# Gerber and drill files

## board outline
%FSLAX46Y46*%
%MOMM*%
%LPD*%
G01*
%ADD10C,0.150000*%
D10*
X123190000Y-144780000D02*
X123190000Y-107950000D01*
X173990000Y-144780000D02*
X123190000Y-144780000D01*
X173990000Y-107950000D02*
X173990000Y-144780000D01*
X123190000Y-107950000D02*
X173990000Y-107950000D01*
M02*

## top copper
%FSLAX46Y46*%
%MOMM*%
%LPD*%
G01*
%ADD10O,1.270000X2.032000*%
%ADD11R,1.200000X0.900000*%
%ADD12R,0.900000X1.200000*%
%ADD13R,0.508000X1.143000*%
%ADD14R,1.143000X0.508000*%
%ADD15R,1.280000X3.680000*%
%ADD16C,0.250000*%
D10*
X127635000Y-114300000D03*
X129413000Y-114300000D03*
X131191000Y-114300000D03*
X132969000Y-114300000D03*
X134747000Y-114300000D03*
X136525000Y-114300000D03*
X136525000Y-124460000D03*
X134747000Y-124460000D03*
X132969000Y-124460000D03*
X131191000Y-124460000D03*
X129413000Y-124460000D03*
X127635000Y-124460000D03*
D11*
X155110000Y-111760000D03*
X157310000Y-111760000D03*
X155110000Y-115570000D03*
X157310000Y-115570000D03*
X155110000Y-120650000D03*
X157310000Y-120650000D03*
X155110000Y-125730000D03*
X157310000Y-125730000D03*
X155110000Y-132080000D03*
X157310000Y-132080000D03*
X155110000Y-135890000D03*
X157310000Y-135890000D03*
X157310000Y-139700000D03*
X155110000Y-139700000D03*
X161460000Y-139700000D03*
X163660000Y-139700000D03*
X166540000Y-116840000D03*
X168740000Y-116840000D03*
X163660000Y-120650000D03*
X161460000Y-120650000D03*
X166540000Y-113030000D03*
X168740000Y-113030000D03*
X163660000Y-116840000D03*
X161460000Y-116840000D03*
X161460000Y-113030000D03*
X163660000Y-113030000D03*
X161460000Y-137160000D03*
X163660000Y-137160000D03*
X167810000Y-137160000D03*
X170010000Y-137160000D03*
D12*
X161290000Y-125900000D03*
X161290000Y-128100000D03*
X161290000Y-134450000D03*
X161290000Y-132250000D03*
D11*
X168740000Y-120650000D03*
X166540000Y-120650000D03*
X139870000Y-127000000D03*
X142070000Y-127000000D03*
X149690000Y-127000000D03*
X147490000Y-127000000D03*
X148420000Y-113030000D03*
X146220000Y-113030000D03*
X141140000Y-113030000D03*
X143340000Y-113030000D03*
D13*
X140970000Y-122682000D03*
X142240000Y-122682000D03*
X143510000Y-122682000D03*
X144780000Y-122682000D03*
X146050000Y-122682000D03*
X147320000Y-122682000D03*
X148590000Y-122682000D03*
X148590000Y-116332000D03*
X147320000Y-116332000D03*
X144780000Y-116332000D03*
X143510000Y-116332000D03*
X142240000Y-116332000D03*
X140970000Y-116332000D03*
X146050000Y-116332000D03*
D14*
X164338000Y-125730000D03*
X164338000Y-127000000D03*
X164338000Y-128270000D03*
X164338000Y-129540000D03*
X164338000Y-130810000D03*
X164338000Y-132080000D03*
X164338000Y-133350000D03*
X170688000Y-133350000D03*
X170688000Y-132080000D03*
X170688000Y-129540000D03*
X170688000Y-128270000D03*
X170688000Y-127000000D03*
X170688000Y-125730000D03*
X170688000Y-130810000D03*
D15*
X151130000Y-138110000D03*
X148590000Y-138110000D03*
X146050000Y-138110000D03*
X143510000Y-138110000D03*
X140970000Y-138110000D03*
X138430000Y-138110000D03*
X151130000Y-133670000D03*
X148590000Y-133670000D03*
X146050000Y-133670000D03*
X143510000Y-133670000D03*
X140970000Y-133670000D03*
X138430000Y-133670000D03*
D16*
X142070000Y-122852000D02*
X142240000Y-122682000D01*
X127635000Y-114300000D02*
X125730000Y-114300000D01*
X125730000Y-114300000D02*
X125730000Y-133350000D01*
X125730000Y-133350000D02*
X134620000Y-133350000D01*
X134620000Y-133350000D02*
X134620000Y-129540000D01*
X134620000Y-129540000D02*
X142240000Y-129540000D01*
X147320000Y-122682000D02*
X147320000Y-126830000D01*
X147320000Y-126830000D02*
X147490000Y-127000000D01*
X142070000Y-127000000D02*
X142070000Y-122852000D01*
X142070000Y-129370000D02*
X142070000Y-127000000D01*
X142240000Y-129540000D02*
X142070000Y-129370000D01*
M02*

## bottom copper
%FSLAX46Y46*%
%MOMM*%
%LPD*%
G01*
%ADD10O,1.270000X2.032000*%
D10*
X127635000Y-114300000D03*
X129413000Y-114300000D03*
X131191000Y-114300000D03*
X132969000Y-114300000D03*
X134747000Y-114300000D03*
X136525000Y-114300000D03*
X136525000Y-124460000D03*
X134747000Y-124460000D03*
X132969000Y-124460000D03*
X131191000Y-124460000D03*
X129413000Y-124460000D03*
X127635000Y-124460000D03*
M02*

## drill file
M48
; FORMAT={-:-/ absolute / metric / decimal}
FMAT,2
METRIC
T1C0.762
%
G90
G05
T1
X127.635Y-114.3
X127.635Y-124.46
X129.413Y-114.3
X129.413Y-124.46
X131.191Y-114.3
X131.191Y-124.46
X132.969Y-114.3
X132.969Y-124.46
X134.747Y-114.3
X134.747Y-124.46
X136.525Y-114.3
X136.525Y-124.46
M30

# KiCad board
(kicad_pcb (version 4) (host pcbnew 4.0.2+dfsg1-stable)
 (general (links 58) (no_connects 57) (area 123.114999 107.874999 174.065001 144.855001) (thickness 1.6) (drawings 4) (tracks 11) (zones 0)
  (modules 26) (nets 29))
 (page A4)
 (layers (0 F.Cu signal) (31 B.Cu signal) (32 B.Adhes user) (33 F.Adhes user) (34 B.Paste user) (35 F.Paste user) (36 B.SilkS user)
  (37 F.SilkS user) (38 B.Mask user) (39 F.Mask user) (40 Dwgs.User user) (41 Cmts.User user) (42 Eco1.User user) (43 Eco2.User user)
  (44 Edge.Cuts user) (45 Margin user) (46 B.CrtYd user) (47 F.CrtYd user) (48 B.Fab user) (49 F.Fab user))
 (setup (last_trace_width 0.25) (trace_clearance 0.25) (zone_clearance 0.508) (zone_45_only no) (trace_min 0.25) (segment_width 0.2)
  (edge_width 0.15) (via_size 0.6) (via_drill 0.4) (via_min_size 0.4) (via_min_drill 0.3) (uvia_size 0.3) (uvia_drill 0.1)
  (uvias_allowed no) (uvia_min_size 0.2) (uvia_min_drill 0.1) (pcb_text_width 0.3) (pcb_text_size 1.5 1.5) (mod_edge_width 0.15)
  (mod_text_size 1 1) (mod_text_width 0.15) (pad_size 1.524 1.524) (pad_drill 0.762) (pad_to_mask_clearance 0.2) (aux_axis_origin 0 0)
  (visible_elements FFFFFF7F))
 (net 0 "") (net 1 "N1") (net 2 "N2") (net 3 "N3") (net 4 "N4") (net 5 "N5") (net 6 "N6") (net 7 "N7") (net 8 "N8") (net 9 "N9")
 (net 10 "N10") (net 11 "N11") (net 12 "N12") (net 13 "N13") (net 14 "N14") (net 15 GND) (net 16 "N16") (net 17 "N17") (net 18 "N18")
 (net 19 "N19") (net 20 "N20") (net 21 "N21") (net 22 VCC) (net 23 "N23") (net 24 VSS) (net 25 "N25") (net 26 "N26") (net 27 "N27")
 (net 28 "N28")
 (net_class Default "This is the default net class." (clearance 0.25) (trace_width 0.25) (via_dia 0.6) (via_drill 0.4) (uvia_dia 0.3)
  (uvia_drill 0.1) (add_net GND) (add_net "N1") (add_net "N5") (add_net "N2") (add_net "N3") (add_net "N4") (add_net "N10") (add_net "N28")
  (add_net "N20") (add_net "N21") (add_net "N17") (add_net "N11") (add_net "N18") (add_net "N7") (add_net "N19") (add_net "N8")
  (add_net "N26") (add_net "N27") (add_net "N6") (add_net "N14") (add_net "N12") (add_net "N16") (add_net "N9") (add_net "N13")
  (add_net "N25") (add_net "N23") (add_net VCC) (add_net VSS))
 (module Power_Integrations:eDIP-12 (layer F.Cu) (at 132.08 119.38)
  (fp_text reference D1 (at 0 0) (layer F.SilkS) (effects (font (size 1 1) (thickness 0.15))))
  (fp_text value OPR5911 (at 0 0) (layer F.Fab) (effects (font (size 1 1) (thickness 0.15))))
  (pad 1 thru_hole oval (at -4.445 -5.08) (size 1.27 2.032) (drill 0.762) (layers *.Cu *.Mask F.SilkS) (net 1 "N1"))
  (pad 2 thru_hole oval (at -2.667 -5.08) (size 1.27 2.032) (drill 0.762) (layers *.Cu *.Mask F.SilkS) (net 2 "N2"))
  (pad 3 thru_hole oval (at -0.889 -5.08) (size 1.27 2.032) (drill 0.762) (layers *.Cu *.Mask F.SilkS))
  (pad 4 thru_hole oval (at 0.889 -5.08) (size 1.27 2.032) (drill 0.762) (layers *.Cu *.Mask F.SilkS))
  (pad 5 thru_hole oval (at 2.667 -5.08) (size 1.27 2.032) (drill 0.762) (layers *.Cu *.Mask F.SilkS))
  (pad 6 thru_hole oval (at 4.445 -5.08) (size 1.27 2.032) (drill 0.762) (layers *.Cu *.Mask F.SilkS) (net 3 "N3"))
  (pad 7 thru_hole oval (at 4.445 5.08) (size 1.27 2.032) (drill 0.762) (layers *.Cu *.Mask F.SilkS) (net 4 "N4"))
  (pad 8 thru_hole oval (at 2.667 5.08) (size 1.27 2.032) (drill 0.762) (layers *.Cu *.Mask F.SilkS))
  (pad 9 thru_hole oval (at 0.889 5.08) (size 1.27 2.032) (drill 0.762) (layers *.Cu *.Mask F.SilkS))
  (pad 10 thru_hole oval (at -0.889 5.08) (size 1.27 2.032) (drill 0.762) (layers *.Cu *.Mask F.SilkS))
  (pad 11 thru_hole oval (at -2.667 5.08) (size 1.27 2.032) (drill 0.762) (layers *.Cu *.Mask F.SilkS))
  (pad 12 thru_hole oval (at -4.445 5.08) (size 1.27 2.032) (drill 0.762) (layers *.Cu *.Mask F.SilkS) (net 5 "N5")))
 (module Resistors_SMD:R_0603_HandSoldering (layer F.Cu) (at 156.21 111.76)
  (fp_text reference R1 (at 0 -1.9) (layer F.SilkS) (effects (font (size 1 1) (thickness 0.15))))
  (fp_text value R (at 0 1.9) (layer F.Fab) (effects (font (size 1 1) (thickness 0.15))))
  (pad 1 smd rect (at -1.1 0) (size 1.2 0.9) (layers F.Cu F.Paste F.Mask) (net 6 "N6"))
  (pad 2 smd rect (at 1.1 0) (size 1.2 0.9) (layers F.Cu F.Paste F.Mask) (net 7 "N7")))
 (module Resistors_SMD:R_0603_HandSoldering (layer F.Cu) (at 156.21 115.57)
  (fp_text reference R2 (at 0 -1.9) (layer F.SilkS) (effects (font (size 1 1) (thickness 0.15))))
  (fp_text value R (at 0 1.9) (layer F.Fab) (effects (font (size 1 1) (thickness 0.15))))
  (pad 1 smd rect (at -1.1 0) (size 1.2 0.9) (layers F.Cu F.Paste F.Mask) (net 6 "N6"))
  (pad 2 smd rect (at 1.1 0) (size 1.2 0.9) (layers F.Cu F.Paste F.Mask) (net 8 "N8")))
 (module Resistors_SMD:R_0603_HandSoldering (layer F.Cu) (at 156.21 120.65)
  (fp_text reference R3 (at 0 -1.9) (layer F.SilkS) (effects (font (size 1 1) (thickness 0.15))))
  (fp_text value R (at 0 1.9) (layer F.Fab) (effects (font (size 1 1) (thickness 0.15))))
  (pad 1 smd rect (at -1.1 0) (size 1.2 0.9) (layers F.Cu F.Paste F.Mask) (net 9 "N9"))
  (pad 2 smd rect (at 1.1 0) (size 1.2 0.9) (layers F.Cu F.Paste F.Mask) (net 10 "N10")))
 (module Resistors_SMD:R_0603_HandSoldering (layer F.Cu) (at 156.21 125.73)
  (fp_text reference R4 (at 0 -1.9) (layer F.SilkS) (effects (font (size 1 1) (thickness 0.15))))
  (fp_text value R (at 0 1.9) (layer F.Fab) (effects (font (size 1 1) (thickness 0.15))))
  (pad 1 smd rect (at -1.1 0) (size 1.2 0.9) (layers F.Cu F.Paste F.Mask) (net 9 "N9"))
  (pad 2 smd rect (at 1.1 0) (size 1.2 0.9) (layers F.Cu F.Paste F.Mask) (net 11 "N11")))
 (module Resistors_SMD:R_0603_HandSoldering (layer F.Cu) (at 156.21 132.08)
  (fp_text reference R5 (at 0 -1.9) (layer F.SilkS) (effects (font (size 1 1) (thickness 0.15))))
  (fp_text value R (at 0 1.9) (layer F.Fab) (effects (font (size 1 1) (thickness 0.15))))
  (pad 1 smd rect (at -1.1 0) (size 1.2 0.9) (layers F.Cu F.Paste F.Mask) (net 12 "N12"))
  (pad 2 smd rect (at 1.1 0) (size 1.2 0.9) (layers F.Cu F.Paste F.Mask) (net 11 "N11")))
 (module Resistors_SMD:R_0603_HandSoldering (layer F.Cu) (at 156.21 135.89)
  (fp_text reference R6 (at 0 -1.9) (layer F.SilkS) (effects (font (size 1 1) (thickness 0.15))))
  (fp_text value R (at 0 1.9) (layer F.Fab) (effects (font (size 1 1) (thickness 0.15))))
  (pad 1 smd rect (at -1.1 0) (size 1.2 0.9) (layers F.Cu F.Paste F.Mask) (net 12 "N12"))
  (pad 2 smd rect (at 1.1 0) (size 1.2 0.9) (layers F.Cu F.Paste F.Mask) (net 7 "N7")))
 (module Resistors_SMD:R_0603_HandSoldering (layer F.Cu) (at 156.21 139.7 180)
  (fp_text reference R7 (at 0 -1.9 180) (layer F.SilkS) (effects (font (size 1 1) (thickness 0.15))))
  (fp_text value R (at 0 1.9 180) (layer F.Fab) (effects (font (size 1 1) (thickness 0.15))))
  (pad 1 smd rect (at -1.1 0 180) (size 1.2 0.9) (layers F.Cu F.Paste F.Mask) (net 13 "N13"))
  (pad 2 smd rect (at 1.1 0 180) (size 1.2 0.9) (layers F.Cu F.Paste F.Mask) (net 8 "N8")))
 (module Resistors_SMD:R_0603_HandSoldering (layer F.Cu) (at 162.56 139.7)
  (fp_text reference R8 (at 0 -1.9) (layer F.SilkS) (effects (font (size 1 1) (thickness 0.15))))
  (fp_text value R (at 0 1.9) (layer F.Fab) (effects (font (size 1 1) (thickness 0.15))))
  (pad 1 smd rect (at -1.1 0) (size 1.2 0.9) (layers F.Cu F.Paste F.Mask) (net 13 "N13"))
  (pad 2 smd rect (at 1.1 0) (size 1.2 0.9) (layers F.Cu F.Paste F.Mask) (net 10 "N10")))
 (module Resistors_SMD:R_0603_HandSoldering (layer F.Cu) (at 167.64 116.84)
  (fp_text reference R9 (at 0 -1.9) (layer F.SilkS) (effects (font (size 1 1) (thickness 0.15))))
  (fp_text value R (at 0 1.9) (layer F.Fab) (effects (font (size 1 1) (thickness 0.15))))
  (pad 1 smd rect (at -1.1 0) (size 1.2 0.9) (layers F.Cu F.Paste F.Mask) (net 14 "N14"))
  (pad 2 smd rect (at 1.1 0) (size 1.2 0.9) (layers F.Cu F.Paste F.Mask) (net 10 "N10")))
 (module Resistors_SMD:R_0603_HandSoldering (layer F.Cu) (at 162.56 120.65 180)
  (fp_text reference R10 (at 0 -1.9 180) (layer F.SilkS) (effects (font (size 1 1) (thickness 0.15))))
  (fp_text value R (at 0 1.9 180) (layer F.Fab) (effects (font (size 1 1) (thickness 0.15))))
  (pad 1 smd rect (at -1.1 0 180) (size 1.2 0.9) (layers F.Cu F.Paste F.Mask) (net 14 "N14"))
  (pad 2 smd rect (at 1.1 0 180) (size 1.2 0.9) (layers F.Cu F.Paste F.Mask) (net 11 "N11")))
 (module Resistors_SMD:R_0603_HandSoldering (layer F.Cu) (at 167.64 113.03)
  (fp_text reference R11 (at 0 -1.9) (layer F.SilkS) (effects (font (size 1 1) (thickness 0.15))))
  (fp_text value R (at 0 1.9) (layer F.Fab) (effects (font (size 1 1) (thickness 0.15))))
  (pad 1 smd rect (at -1.1 0) (size 1.2 0.9) (layers F.Cu F.Paste F.Mask) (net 14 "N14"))
  (pad 2 smd rect (at 1.1 0) (size 1.2 0.9) (layers F.Cu F.Paste F.Mask) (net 7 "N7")))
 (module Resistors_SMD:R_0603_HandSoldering (layer F.Cu) (at 162.56 116.84 180)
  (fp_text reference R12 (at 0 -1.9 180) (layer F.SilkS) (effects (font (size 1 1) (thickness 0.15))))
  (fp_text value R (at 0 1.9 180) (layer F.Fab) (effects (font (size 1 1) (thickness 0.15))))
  (pad 1 smd rect (at -1.1 0 180) (size 1.2 0.9) (layers F.Cu F.Paste F.Mask) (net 14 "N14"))
  (pad 2 smd rect (at 1.1 0 180) (size 1.2 0.9) (layers F.Cu F.Paste F.Mask) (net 8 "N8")))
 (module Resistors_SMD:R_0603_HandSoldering (layer F.Cu) (at 162.56 113.03)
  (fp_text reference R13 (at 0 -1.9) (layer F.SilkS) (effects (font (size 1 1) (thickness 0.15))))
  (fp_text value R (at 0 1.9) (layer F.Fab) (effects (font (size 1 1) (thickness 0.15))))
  (pad 1 smd rect (at -1.1 0) (size 1.2 0.9) (layers F.Cu F.Paste F.Mask) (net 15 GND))
  (pad 2 smd rect (at 1.1 0) (size 1.2 0.9) (layers F.Cu F.Paste F.Mask) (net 6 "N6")))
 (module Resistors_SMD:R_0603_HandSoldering (layer F.Cu) (at 162.56 137.16)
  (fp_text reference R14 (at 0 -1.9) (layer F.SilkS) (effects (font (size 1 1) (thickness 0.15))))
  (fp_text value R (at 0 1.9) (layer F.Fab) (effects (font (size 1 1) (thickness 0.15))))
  (pad 1 smd rect (at -1.1 0) (size 1.2 0.9) (layers F.Cu F.Paste F.Mask) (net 15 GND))
  (pad 2 smd rect (at 1.1 0) (size 1.2 0.9) (layers F.Cu F.Paste F.Mask) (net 12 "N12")))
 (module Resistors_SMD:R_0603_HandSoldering (layer F.Cu) (at 168.91 137.16)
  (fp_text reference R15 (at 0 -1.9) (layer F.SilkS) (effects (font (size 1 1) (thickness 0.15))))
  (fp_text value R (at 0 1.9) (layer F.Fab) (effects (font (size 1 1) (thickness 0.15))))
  (pad 1 smd rect (at -1.1 0) (size 1.2 0.9) (layers F.Cu F.Paste F.Mask) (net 15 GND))
  (pad 2 smd rect (at 1.1 0) (size 1.2 0.9) (layers F.Cu F.Paste F.Mask) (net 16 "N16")))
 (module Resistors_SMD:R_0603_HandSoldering (layer F.Cu) (at 161.29 127 270)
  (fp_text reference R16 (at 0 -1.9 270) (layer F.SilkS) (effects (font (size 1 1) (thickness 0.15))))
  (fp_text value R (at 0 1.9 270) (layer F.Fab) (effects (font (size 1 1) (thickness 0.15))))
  (pad 1 smd rect (at -1.1 0 270) (size 1.2 0.9) (layers F.Cu F.Paste F.Mask) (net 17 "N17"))
  (pad 2 smd rect (at 1.1 0 270) (size 1.2 0.9) (layers F.Cu F.Paste F.Mask) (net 9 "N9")))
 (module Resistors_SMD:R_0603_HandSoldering (layer F.Cu) (at 161.29 133.35 90)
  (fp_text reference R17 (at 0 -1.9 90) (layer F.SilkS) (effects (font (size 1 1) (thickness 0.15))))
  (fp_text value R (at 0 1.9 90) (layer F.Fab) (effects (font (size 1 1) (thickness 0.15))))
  (pad 1 smd rect (at -1.1 0 90) (size 1.2 0.9) (layers F.Cu F.Paste F.Mask) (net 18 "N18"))
  (pad 2 smd rect (at 1.1 0 90) (size 1.2 0.9) (layers F.Cu F.Paste F.Mask) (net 13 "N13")))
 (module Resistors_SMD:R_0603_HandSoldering (layer F.Cu) (at 167.64 120.65 180)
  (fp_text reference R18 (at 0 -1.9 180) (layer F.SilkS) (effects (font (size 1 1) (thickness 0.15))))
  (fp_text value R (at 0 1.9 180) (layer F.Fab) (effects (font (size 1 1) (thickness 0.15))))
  (pad 1 smd rect (at -1.1 0 180) (size 1.2 0.9) (layers F.Cu F.Paste F.Mask) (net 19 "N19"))
  (pad 2 smd rect (at 1.1 0 180) (size 1.2 0.9) (layers F.Cu F.Paste F.Mask) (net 14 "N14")))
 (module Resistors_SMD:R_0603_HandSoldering (layer F.Cu) (at 140.97 127)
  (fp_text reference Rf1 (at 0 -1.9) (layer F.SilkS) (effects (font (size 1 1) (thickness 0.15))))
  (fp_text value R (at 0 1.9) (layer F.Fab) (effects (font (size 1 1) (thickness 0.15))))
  (pad 1 smd rect (at -1.1 0) (size 1.2 0.9) (layers F.Cu F.Paste F.Mask) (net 1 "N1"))
  (pad 2 smd rect (at 1.1 0) (size 1.2 0.9) (layers F.Cu F.Paste F.Mask) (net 10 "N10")))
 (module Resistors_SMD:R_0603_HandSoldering (layer F.Cu) (at 148.59 127 180)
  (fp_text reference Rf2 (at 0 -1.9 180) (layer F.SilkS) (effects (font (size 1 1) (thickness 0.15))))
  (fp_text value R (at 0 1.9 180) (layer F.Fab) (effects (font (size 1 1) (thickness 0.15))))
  (pad 1 smd rect (at -1.1 0 180) (size 1.2 0.9) (layers F.Cu F.Paste F.Mask) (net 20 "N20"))
  (pad 2 smd rect (at 1.1 0 180) (size 1.2 0.9) (layers F.Cu F.Paste F.Mask) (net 3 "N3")))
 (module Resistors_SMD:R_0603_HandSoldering (layer F.Cu) (at 147.32 113.03 180)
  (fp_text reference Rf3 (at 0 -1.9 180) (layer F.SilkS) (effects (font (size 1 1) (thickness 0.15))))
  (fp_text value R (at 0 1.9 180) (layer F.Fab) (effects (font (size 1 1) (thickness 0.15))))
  (pad 1 smd rect (at -1.1 0 180) (size 1.2 0.9) (layers F.Cu F.Paste F.Mask) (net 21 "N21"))
  (pad 2 smd rect (at 1.1 0 180) (size 1.2 0.9) (layers F.Cu F.Paste F.Mask) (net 4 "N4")))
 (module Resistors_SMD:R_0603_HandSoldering (layer F.Cu) (at 142.24 113.03)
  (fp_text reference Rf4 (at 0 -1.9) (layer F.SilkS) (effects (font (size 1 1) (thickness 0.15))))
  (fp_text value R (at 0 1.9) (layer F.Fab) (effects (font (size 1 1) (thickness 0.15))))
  (pad 1 smd rect (at -1.1 0) (size 1.2 0.9) (layers F.Cu F.Paste F.Mask) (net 5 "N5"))
  (pad 2 smd rect (at 1.1 0) (size 1.2 0.9) (layers F.Cu F.Paste F.Mask) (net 17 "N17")))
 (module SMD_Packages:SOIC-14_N (layer F.Cu) (at 144.78 119.38)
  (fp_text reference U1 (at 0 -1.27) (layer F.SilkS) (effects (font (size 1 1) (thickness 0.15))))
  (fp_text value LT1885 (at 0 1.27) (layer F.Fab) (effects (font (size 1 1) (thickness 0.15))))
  (pad 1 smd rect (at -3.81 3.302) (size 0.508 1.143) (layers F.Cu F.Paste F.Mask) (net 10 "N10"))
  (pad 2 smd rect (at -2.54 3.302) (size 0.508 1.143) (layers F.Cu F.Paste F.Mask) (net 1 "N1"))
  (pad 3 smd rect (at -1.27 3.302) (size 0.508 1.143) (layers F.Cu F.Paste F.Mask) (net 15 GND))
  (pad 4 smd rect (at 0 3.302) (size 0.508 1.143) (layers F.Cu F.Paste F.Mask) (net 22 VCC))
  (pad 5 smd rect (at 1.27 3.302) (size 0.508 1.143) (layers F.Cu F.Paste F.Mask) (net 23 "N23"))
  (pad 6 smd rect (at 2.54 3.302) (size 0.508 1.143) (layers F.Cu F.Paste F.Mask) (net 3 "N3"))
  (pad 7 smd rect (at 3.81 3.302) (size 0.508 1.143) (layers F.Cu F.Paste F.Mask) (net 20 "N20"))
  (pad 8 smd rect (at 3.81 -3.048) (size 0.508 1.143) (layers F.Cu F.Paste F.Mask) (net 21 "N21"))
  (pad 9 smd rect (at 2.54 -3.048) (size 0.508 1.143) (layers F.Cu F.Paste F.Mask) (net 4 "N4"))
  (pad 11 smd rect (at 0 -3.048) (size 0.508 1.143) (layers F.Cu F.Paste F.Mask) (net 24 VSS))
  (pad 12 smd rect (at -1.27 -3.048) (size 0.508 1.143) (layers F.Cu F.Paste F.Mask) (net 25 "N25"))
  (pad 13 smd rect (at -2.54 -3.048) (size 0.508 1.143) (layers F.Cu F.Paste F.Mask) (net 5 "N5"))
  (pad 14 smd rect (at -3.81 -3.048) (size 0.508 1.143) (layers F.Cu F.Paste F.Mask) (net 17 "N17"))
  (pad 10 smd rect (at 1.27 -3.048) (size 0.508 1.143) (layers F.Cu F.Paste F.Mask) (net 15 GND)))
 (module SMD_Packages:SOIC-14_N (layer F.Cu) (at 167.64 129.54 270)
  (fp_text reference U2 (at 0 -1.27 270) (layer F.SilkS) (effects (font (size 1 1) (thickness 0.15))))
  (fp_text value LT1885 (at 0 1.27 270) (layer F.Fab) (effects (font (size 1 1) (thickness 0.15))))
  (pad 1 smd rect (at -3.81 3.302 270) (size 0.508 1.143) (layers F.Cu F.Paste F.Mask) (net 17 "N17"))
  (pad 2 smd rect (at -2.54 3.302 270) (size 0.508 1.143) (layers F.Cu F.Paste F.Mask) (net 9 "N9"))
  (pad 3 smd rect (at -1.27 3.302 270) (size 0.508 1.143) (layers F.Cu F.Paste F.Mask) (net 6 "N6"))
  (pad 4 smd rect (at 0 3.302 270) (size 0.508 1.143) (layers F.Cu F.Paste F.Mask) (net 22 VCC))
  (pad 5 smd rect (at 1.27 3.302 270) (size 0.508 1.143) (layers F.Cu F.Paste F.Mask) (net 12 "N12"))
  (pad 6 smd rect (at 2.54 3.302 270) (size 0.508 1.143) (layers F.Cu F.Paste F.Mask) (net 13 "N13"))
  (pad 7 smd rect (at 3.81 3.302 270) (size 0.508 1.143) (layers F.Cu F.Paste F.Mask) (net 18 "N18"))
  (pad 8 smd rect (at 3.81 -3.048 270) (size 0.508 1.143) (layers F.Cu F.Paste F.Mask) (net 19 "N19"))
  (pad 9 smd rect (at 2.54 -3.048 270) (size 0.508 1.143) (layers F.Cu F.Paste F.Mask) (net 14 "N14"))
  (pad 11 smd rect (at 0 -3.048 270) (size 0.508 1.143) (layers F.Cu F.Paste F.Mask) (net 24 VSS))
  (pad 12 smd rect (at -1.27 -3.048 270) (size 0.508 1.143) (layers F.Cu F.Paste F.Mask))
  (pad 13 smd rect (at -2.54 -3.048 270) (size 0.508 1.143) (layers F.Cu F.Paste F.Mask))
  (pad 14 smd rect (at -3.81 -3.048 270) (size 0.508 1.143) (layers F.Cu F.Paste F.Mask))
  (pad 10 smd rect (at 1.27 -3.048 270) (size 0.508 1.143) (layers F.Cu F.Paste F.Mask) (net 16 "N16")))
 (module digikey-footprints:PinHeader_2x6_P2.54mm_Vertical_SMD (layer F.Cu) (at 144.78 135.89 180)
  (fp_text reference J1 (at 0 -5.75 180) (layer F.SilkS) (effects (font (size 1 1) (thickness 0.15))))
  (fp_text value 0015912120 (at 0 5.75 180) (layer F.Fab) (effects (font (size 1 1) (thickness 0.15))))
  (pad 1 smd rect (at -6.35 -2.22 180) (size 1.28 3.68) (layers F.Cu F.Paste F.Mask) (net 10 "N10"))
  (pad 2 smd rect (at -3.81 -2.22 180) (size 1.28 3.68) (layers F.Cu F.Paste F.Mask) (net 17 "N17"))
  (pad 3 smd rect (at -1.27 -2.22 180) (size 1.28 3.68) (layers F.Cu F.Paste F.Mask) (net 24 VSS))
  (pad 4 smd rect (at 1.27 -2.22 180) (size 1.28 3.68) (layers F.Cu F.Paste F.Mask) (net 18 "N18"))
  (pad 5 smd rect (at 3.81 -2.22 180) (size 1.28 3.68) (layers F.Cu F.Paste F.Mask) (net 15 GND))
  (pad 6 smd rect (at 6.35 -2.22 180) (size 1.28 3.68) (layers F.Cu F.Paste F.Mask) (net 19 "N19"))
  (pad 7 smd rect (at -6.35 2.22 180) (size 1.28 3.68) (layers F.Cu F.Paste F.Mask) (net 22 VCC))
  (pad 8 smd rect (at -3.81 2.22 180) (size 1.28 3.68) (layers F.Cu F.Paste F.Mask) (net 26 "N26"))
  (pad 9 smd rect (at -1.27 2.22 180) (size 1.28 3.68) (layers F.Cu F.Paste F.Mask) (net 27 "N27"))
  (pad 10 smd rect (at 1.27 2.22 180) (size 1.28 3.68) (layers F.Cu F.Paste F.Mask) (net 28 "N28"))
  (pad 11 smd rect (at 3.81 2.22 180) (size 1.28 3.68) (layers F.Cu F.Paste F.Mask) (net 20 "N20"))
  (pad 12 smd rect (at 6.35 2.22 180) (size 1.28 3.68) (layers F.Cu F.Paste F.Mask) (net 21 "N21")))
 (gr_line (start 123.19 144.78) (end 123.19 107.95) (angle 90) (layer Edge.Cuts) (width 0.15))
 (gr_line (start 173.99 144.78) (end 123.19 144.78) (angle 90) (layer Edge.Cuts) (width 0.15))
 (gr_line (start 173.99 107.95) (end 173.99 144.78) (angle 90) (layer Edge.Cuts) (width 0.15))
 (gr_line (start 123.19 107.95) (end 173.99 107.95) (angle 90) (layer Edge.Cuts) (width 0.15))
 (segment (start 142.07 122.852) (end 142.24 122.682) (width 0.25) (layer F.Cu) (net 1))
 (segment (start 127.635 114.3) (end 125.73 114.3) (width 0.25) (layer F.Cu) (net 1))
 (segment (start 125.73 114.3) (end 125.73 133.35) (width 0.25) (layer F.Cu) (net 1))
 (segment (start 125.73 133.35) (end 134.62 133.35) (width 0.25) (layer F.Cu) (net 1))
 (segment (start 134.62 133.35) (end 134.62 129.54) (width 0.25) (layer F.Cu) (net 1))
 (segment (start 134.62 129.54) (end 142.24 129.54) (width 0.25) (layer F.Cu) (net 1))
 (segment (start 147.32 122.682) (end 147.32 126.83) (width 0.25) (layer F.Cu) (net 3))
 (segment (start 147.32 126.83) (end 147.49 127) (width 0.25) (layer F.Cu) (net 3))
 (segment (start 142.07 127) (end 142.07 122.852) (width 0.25) (layer F.Cu) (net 10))
 (segment (start 142.07 129.37) (end 142.07 127) (width 0.25) (layer F.Cu) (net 10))
 (segment (start 142.24 129.54) (end 142.07 129.37) (width 0.25) (layer F.Cu) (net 10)))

